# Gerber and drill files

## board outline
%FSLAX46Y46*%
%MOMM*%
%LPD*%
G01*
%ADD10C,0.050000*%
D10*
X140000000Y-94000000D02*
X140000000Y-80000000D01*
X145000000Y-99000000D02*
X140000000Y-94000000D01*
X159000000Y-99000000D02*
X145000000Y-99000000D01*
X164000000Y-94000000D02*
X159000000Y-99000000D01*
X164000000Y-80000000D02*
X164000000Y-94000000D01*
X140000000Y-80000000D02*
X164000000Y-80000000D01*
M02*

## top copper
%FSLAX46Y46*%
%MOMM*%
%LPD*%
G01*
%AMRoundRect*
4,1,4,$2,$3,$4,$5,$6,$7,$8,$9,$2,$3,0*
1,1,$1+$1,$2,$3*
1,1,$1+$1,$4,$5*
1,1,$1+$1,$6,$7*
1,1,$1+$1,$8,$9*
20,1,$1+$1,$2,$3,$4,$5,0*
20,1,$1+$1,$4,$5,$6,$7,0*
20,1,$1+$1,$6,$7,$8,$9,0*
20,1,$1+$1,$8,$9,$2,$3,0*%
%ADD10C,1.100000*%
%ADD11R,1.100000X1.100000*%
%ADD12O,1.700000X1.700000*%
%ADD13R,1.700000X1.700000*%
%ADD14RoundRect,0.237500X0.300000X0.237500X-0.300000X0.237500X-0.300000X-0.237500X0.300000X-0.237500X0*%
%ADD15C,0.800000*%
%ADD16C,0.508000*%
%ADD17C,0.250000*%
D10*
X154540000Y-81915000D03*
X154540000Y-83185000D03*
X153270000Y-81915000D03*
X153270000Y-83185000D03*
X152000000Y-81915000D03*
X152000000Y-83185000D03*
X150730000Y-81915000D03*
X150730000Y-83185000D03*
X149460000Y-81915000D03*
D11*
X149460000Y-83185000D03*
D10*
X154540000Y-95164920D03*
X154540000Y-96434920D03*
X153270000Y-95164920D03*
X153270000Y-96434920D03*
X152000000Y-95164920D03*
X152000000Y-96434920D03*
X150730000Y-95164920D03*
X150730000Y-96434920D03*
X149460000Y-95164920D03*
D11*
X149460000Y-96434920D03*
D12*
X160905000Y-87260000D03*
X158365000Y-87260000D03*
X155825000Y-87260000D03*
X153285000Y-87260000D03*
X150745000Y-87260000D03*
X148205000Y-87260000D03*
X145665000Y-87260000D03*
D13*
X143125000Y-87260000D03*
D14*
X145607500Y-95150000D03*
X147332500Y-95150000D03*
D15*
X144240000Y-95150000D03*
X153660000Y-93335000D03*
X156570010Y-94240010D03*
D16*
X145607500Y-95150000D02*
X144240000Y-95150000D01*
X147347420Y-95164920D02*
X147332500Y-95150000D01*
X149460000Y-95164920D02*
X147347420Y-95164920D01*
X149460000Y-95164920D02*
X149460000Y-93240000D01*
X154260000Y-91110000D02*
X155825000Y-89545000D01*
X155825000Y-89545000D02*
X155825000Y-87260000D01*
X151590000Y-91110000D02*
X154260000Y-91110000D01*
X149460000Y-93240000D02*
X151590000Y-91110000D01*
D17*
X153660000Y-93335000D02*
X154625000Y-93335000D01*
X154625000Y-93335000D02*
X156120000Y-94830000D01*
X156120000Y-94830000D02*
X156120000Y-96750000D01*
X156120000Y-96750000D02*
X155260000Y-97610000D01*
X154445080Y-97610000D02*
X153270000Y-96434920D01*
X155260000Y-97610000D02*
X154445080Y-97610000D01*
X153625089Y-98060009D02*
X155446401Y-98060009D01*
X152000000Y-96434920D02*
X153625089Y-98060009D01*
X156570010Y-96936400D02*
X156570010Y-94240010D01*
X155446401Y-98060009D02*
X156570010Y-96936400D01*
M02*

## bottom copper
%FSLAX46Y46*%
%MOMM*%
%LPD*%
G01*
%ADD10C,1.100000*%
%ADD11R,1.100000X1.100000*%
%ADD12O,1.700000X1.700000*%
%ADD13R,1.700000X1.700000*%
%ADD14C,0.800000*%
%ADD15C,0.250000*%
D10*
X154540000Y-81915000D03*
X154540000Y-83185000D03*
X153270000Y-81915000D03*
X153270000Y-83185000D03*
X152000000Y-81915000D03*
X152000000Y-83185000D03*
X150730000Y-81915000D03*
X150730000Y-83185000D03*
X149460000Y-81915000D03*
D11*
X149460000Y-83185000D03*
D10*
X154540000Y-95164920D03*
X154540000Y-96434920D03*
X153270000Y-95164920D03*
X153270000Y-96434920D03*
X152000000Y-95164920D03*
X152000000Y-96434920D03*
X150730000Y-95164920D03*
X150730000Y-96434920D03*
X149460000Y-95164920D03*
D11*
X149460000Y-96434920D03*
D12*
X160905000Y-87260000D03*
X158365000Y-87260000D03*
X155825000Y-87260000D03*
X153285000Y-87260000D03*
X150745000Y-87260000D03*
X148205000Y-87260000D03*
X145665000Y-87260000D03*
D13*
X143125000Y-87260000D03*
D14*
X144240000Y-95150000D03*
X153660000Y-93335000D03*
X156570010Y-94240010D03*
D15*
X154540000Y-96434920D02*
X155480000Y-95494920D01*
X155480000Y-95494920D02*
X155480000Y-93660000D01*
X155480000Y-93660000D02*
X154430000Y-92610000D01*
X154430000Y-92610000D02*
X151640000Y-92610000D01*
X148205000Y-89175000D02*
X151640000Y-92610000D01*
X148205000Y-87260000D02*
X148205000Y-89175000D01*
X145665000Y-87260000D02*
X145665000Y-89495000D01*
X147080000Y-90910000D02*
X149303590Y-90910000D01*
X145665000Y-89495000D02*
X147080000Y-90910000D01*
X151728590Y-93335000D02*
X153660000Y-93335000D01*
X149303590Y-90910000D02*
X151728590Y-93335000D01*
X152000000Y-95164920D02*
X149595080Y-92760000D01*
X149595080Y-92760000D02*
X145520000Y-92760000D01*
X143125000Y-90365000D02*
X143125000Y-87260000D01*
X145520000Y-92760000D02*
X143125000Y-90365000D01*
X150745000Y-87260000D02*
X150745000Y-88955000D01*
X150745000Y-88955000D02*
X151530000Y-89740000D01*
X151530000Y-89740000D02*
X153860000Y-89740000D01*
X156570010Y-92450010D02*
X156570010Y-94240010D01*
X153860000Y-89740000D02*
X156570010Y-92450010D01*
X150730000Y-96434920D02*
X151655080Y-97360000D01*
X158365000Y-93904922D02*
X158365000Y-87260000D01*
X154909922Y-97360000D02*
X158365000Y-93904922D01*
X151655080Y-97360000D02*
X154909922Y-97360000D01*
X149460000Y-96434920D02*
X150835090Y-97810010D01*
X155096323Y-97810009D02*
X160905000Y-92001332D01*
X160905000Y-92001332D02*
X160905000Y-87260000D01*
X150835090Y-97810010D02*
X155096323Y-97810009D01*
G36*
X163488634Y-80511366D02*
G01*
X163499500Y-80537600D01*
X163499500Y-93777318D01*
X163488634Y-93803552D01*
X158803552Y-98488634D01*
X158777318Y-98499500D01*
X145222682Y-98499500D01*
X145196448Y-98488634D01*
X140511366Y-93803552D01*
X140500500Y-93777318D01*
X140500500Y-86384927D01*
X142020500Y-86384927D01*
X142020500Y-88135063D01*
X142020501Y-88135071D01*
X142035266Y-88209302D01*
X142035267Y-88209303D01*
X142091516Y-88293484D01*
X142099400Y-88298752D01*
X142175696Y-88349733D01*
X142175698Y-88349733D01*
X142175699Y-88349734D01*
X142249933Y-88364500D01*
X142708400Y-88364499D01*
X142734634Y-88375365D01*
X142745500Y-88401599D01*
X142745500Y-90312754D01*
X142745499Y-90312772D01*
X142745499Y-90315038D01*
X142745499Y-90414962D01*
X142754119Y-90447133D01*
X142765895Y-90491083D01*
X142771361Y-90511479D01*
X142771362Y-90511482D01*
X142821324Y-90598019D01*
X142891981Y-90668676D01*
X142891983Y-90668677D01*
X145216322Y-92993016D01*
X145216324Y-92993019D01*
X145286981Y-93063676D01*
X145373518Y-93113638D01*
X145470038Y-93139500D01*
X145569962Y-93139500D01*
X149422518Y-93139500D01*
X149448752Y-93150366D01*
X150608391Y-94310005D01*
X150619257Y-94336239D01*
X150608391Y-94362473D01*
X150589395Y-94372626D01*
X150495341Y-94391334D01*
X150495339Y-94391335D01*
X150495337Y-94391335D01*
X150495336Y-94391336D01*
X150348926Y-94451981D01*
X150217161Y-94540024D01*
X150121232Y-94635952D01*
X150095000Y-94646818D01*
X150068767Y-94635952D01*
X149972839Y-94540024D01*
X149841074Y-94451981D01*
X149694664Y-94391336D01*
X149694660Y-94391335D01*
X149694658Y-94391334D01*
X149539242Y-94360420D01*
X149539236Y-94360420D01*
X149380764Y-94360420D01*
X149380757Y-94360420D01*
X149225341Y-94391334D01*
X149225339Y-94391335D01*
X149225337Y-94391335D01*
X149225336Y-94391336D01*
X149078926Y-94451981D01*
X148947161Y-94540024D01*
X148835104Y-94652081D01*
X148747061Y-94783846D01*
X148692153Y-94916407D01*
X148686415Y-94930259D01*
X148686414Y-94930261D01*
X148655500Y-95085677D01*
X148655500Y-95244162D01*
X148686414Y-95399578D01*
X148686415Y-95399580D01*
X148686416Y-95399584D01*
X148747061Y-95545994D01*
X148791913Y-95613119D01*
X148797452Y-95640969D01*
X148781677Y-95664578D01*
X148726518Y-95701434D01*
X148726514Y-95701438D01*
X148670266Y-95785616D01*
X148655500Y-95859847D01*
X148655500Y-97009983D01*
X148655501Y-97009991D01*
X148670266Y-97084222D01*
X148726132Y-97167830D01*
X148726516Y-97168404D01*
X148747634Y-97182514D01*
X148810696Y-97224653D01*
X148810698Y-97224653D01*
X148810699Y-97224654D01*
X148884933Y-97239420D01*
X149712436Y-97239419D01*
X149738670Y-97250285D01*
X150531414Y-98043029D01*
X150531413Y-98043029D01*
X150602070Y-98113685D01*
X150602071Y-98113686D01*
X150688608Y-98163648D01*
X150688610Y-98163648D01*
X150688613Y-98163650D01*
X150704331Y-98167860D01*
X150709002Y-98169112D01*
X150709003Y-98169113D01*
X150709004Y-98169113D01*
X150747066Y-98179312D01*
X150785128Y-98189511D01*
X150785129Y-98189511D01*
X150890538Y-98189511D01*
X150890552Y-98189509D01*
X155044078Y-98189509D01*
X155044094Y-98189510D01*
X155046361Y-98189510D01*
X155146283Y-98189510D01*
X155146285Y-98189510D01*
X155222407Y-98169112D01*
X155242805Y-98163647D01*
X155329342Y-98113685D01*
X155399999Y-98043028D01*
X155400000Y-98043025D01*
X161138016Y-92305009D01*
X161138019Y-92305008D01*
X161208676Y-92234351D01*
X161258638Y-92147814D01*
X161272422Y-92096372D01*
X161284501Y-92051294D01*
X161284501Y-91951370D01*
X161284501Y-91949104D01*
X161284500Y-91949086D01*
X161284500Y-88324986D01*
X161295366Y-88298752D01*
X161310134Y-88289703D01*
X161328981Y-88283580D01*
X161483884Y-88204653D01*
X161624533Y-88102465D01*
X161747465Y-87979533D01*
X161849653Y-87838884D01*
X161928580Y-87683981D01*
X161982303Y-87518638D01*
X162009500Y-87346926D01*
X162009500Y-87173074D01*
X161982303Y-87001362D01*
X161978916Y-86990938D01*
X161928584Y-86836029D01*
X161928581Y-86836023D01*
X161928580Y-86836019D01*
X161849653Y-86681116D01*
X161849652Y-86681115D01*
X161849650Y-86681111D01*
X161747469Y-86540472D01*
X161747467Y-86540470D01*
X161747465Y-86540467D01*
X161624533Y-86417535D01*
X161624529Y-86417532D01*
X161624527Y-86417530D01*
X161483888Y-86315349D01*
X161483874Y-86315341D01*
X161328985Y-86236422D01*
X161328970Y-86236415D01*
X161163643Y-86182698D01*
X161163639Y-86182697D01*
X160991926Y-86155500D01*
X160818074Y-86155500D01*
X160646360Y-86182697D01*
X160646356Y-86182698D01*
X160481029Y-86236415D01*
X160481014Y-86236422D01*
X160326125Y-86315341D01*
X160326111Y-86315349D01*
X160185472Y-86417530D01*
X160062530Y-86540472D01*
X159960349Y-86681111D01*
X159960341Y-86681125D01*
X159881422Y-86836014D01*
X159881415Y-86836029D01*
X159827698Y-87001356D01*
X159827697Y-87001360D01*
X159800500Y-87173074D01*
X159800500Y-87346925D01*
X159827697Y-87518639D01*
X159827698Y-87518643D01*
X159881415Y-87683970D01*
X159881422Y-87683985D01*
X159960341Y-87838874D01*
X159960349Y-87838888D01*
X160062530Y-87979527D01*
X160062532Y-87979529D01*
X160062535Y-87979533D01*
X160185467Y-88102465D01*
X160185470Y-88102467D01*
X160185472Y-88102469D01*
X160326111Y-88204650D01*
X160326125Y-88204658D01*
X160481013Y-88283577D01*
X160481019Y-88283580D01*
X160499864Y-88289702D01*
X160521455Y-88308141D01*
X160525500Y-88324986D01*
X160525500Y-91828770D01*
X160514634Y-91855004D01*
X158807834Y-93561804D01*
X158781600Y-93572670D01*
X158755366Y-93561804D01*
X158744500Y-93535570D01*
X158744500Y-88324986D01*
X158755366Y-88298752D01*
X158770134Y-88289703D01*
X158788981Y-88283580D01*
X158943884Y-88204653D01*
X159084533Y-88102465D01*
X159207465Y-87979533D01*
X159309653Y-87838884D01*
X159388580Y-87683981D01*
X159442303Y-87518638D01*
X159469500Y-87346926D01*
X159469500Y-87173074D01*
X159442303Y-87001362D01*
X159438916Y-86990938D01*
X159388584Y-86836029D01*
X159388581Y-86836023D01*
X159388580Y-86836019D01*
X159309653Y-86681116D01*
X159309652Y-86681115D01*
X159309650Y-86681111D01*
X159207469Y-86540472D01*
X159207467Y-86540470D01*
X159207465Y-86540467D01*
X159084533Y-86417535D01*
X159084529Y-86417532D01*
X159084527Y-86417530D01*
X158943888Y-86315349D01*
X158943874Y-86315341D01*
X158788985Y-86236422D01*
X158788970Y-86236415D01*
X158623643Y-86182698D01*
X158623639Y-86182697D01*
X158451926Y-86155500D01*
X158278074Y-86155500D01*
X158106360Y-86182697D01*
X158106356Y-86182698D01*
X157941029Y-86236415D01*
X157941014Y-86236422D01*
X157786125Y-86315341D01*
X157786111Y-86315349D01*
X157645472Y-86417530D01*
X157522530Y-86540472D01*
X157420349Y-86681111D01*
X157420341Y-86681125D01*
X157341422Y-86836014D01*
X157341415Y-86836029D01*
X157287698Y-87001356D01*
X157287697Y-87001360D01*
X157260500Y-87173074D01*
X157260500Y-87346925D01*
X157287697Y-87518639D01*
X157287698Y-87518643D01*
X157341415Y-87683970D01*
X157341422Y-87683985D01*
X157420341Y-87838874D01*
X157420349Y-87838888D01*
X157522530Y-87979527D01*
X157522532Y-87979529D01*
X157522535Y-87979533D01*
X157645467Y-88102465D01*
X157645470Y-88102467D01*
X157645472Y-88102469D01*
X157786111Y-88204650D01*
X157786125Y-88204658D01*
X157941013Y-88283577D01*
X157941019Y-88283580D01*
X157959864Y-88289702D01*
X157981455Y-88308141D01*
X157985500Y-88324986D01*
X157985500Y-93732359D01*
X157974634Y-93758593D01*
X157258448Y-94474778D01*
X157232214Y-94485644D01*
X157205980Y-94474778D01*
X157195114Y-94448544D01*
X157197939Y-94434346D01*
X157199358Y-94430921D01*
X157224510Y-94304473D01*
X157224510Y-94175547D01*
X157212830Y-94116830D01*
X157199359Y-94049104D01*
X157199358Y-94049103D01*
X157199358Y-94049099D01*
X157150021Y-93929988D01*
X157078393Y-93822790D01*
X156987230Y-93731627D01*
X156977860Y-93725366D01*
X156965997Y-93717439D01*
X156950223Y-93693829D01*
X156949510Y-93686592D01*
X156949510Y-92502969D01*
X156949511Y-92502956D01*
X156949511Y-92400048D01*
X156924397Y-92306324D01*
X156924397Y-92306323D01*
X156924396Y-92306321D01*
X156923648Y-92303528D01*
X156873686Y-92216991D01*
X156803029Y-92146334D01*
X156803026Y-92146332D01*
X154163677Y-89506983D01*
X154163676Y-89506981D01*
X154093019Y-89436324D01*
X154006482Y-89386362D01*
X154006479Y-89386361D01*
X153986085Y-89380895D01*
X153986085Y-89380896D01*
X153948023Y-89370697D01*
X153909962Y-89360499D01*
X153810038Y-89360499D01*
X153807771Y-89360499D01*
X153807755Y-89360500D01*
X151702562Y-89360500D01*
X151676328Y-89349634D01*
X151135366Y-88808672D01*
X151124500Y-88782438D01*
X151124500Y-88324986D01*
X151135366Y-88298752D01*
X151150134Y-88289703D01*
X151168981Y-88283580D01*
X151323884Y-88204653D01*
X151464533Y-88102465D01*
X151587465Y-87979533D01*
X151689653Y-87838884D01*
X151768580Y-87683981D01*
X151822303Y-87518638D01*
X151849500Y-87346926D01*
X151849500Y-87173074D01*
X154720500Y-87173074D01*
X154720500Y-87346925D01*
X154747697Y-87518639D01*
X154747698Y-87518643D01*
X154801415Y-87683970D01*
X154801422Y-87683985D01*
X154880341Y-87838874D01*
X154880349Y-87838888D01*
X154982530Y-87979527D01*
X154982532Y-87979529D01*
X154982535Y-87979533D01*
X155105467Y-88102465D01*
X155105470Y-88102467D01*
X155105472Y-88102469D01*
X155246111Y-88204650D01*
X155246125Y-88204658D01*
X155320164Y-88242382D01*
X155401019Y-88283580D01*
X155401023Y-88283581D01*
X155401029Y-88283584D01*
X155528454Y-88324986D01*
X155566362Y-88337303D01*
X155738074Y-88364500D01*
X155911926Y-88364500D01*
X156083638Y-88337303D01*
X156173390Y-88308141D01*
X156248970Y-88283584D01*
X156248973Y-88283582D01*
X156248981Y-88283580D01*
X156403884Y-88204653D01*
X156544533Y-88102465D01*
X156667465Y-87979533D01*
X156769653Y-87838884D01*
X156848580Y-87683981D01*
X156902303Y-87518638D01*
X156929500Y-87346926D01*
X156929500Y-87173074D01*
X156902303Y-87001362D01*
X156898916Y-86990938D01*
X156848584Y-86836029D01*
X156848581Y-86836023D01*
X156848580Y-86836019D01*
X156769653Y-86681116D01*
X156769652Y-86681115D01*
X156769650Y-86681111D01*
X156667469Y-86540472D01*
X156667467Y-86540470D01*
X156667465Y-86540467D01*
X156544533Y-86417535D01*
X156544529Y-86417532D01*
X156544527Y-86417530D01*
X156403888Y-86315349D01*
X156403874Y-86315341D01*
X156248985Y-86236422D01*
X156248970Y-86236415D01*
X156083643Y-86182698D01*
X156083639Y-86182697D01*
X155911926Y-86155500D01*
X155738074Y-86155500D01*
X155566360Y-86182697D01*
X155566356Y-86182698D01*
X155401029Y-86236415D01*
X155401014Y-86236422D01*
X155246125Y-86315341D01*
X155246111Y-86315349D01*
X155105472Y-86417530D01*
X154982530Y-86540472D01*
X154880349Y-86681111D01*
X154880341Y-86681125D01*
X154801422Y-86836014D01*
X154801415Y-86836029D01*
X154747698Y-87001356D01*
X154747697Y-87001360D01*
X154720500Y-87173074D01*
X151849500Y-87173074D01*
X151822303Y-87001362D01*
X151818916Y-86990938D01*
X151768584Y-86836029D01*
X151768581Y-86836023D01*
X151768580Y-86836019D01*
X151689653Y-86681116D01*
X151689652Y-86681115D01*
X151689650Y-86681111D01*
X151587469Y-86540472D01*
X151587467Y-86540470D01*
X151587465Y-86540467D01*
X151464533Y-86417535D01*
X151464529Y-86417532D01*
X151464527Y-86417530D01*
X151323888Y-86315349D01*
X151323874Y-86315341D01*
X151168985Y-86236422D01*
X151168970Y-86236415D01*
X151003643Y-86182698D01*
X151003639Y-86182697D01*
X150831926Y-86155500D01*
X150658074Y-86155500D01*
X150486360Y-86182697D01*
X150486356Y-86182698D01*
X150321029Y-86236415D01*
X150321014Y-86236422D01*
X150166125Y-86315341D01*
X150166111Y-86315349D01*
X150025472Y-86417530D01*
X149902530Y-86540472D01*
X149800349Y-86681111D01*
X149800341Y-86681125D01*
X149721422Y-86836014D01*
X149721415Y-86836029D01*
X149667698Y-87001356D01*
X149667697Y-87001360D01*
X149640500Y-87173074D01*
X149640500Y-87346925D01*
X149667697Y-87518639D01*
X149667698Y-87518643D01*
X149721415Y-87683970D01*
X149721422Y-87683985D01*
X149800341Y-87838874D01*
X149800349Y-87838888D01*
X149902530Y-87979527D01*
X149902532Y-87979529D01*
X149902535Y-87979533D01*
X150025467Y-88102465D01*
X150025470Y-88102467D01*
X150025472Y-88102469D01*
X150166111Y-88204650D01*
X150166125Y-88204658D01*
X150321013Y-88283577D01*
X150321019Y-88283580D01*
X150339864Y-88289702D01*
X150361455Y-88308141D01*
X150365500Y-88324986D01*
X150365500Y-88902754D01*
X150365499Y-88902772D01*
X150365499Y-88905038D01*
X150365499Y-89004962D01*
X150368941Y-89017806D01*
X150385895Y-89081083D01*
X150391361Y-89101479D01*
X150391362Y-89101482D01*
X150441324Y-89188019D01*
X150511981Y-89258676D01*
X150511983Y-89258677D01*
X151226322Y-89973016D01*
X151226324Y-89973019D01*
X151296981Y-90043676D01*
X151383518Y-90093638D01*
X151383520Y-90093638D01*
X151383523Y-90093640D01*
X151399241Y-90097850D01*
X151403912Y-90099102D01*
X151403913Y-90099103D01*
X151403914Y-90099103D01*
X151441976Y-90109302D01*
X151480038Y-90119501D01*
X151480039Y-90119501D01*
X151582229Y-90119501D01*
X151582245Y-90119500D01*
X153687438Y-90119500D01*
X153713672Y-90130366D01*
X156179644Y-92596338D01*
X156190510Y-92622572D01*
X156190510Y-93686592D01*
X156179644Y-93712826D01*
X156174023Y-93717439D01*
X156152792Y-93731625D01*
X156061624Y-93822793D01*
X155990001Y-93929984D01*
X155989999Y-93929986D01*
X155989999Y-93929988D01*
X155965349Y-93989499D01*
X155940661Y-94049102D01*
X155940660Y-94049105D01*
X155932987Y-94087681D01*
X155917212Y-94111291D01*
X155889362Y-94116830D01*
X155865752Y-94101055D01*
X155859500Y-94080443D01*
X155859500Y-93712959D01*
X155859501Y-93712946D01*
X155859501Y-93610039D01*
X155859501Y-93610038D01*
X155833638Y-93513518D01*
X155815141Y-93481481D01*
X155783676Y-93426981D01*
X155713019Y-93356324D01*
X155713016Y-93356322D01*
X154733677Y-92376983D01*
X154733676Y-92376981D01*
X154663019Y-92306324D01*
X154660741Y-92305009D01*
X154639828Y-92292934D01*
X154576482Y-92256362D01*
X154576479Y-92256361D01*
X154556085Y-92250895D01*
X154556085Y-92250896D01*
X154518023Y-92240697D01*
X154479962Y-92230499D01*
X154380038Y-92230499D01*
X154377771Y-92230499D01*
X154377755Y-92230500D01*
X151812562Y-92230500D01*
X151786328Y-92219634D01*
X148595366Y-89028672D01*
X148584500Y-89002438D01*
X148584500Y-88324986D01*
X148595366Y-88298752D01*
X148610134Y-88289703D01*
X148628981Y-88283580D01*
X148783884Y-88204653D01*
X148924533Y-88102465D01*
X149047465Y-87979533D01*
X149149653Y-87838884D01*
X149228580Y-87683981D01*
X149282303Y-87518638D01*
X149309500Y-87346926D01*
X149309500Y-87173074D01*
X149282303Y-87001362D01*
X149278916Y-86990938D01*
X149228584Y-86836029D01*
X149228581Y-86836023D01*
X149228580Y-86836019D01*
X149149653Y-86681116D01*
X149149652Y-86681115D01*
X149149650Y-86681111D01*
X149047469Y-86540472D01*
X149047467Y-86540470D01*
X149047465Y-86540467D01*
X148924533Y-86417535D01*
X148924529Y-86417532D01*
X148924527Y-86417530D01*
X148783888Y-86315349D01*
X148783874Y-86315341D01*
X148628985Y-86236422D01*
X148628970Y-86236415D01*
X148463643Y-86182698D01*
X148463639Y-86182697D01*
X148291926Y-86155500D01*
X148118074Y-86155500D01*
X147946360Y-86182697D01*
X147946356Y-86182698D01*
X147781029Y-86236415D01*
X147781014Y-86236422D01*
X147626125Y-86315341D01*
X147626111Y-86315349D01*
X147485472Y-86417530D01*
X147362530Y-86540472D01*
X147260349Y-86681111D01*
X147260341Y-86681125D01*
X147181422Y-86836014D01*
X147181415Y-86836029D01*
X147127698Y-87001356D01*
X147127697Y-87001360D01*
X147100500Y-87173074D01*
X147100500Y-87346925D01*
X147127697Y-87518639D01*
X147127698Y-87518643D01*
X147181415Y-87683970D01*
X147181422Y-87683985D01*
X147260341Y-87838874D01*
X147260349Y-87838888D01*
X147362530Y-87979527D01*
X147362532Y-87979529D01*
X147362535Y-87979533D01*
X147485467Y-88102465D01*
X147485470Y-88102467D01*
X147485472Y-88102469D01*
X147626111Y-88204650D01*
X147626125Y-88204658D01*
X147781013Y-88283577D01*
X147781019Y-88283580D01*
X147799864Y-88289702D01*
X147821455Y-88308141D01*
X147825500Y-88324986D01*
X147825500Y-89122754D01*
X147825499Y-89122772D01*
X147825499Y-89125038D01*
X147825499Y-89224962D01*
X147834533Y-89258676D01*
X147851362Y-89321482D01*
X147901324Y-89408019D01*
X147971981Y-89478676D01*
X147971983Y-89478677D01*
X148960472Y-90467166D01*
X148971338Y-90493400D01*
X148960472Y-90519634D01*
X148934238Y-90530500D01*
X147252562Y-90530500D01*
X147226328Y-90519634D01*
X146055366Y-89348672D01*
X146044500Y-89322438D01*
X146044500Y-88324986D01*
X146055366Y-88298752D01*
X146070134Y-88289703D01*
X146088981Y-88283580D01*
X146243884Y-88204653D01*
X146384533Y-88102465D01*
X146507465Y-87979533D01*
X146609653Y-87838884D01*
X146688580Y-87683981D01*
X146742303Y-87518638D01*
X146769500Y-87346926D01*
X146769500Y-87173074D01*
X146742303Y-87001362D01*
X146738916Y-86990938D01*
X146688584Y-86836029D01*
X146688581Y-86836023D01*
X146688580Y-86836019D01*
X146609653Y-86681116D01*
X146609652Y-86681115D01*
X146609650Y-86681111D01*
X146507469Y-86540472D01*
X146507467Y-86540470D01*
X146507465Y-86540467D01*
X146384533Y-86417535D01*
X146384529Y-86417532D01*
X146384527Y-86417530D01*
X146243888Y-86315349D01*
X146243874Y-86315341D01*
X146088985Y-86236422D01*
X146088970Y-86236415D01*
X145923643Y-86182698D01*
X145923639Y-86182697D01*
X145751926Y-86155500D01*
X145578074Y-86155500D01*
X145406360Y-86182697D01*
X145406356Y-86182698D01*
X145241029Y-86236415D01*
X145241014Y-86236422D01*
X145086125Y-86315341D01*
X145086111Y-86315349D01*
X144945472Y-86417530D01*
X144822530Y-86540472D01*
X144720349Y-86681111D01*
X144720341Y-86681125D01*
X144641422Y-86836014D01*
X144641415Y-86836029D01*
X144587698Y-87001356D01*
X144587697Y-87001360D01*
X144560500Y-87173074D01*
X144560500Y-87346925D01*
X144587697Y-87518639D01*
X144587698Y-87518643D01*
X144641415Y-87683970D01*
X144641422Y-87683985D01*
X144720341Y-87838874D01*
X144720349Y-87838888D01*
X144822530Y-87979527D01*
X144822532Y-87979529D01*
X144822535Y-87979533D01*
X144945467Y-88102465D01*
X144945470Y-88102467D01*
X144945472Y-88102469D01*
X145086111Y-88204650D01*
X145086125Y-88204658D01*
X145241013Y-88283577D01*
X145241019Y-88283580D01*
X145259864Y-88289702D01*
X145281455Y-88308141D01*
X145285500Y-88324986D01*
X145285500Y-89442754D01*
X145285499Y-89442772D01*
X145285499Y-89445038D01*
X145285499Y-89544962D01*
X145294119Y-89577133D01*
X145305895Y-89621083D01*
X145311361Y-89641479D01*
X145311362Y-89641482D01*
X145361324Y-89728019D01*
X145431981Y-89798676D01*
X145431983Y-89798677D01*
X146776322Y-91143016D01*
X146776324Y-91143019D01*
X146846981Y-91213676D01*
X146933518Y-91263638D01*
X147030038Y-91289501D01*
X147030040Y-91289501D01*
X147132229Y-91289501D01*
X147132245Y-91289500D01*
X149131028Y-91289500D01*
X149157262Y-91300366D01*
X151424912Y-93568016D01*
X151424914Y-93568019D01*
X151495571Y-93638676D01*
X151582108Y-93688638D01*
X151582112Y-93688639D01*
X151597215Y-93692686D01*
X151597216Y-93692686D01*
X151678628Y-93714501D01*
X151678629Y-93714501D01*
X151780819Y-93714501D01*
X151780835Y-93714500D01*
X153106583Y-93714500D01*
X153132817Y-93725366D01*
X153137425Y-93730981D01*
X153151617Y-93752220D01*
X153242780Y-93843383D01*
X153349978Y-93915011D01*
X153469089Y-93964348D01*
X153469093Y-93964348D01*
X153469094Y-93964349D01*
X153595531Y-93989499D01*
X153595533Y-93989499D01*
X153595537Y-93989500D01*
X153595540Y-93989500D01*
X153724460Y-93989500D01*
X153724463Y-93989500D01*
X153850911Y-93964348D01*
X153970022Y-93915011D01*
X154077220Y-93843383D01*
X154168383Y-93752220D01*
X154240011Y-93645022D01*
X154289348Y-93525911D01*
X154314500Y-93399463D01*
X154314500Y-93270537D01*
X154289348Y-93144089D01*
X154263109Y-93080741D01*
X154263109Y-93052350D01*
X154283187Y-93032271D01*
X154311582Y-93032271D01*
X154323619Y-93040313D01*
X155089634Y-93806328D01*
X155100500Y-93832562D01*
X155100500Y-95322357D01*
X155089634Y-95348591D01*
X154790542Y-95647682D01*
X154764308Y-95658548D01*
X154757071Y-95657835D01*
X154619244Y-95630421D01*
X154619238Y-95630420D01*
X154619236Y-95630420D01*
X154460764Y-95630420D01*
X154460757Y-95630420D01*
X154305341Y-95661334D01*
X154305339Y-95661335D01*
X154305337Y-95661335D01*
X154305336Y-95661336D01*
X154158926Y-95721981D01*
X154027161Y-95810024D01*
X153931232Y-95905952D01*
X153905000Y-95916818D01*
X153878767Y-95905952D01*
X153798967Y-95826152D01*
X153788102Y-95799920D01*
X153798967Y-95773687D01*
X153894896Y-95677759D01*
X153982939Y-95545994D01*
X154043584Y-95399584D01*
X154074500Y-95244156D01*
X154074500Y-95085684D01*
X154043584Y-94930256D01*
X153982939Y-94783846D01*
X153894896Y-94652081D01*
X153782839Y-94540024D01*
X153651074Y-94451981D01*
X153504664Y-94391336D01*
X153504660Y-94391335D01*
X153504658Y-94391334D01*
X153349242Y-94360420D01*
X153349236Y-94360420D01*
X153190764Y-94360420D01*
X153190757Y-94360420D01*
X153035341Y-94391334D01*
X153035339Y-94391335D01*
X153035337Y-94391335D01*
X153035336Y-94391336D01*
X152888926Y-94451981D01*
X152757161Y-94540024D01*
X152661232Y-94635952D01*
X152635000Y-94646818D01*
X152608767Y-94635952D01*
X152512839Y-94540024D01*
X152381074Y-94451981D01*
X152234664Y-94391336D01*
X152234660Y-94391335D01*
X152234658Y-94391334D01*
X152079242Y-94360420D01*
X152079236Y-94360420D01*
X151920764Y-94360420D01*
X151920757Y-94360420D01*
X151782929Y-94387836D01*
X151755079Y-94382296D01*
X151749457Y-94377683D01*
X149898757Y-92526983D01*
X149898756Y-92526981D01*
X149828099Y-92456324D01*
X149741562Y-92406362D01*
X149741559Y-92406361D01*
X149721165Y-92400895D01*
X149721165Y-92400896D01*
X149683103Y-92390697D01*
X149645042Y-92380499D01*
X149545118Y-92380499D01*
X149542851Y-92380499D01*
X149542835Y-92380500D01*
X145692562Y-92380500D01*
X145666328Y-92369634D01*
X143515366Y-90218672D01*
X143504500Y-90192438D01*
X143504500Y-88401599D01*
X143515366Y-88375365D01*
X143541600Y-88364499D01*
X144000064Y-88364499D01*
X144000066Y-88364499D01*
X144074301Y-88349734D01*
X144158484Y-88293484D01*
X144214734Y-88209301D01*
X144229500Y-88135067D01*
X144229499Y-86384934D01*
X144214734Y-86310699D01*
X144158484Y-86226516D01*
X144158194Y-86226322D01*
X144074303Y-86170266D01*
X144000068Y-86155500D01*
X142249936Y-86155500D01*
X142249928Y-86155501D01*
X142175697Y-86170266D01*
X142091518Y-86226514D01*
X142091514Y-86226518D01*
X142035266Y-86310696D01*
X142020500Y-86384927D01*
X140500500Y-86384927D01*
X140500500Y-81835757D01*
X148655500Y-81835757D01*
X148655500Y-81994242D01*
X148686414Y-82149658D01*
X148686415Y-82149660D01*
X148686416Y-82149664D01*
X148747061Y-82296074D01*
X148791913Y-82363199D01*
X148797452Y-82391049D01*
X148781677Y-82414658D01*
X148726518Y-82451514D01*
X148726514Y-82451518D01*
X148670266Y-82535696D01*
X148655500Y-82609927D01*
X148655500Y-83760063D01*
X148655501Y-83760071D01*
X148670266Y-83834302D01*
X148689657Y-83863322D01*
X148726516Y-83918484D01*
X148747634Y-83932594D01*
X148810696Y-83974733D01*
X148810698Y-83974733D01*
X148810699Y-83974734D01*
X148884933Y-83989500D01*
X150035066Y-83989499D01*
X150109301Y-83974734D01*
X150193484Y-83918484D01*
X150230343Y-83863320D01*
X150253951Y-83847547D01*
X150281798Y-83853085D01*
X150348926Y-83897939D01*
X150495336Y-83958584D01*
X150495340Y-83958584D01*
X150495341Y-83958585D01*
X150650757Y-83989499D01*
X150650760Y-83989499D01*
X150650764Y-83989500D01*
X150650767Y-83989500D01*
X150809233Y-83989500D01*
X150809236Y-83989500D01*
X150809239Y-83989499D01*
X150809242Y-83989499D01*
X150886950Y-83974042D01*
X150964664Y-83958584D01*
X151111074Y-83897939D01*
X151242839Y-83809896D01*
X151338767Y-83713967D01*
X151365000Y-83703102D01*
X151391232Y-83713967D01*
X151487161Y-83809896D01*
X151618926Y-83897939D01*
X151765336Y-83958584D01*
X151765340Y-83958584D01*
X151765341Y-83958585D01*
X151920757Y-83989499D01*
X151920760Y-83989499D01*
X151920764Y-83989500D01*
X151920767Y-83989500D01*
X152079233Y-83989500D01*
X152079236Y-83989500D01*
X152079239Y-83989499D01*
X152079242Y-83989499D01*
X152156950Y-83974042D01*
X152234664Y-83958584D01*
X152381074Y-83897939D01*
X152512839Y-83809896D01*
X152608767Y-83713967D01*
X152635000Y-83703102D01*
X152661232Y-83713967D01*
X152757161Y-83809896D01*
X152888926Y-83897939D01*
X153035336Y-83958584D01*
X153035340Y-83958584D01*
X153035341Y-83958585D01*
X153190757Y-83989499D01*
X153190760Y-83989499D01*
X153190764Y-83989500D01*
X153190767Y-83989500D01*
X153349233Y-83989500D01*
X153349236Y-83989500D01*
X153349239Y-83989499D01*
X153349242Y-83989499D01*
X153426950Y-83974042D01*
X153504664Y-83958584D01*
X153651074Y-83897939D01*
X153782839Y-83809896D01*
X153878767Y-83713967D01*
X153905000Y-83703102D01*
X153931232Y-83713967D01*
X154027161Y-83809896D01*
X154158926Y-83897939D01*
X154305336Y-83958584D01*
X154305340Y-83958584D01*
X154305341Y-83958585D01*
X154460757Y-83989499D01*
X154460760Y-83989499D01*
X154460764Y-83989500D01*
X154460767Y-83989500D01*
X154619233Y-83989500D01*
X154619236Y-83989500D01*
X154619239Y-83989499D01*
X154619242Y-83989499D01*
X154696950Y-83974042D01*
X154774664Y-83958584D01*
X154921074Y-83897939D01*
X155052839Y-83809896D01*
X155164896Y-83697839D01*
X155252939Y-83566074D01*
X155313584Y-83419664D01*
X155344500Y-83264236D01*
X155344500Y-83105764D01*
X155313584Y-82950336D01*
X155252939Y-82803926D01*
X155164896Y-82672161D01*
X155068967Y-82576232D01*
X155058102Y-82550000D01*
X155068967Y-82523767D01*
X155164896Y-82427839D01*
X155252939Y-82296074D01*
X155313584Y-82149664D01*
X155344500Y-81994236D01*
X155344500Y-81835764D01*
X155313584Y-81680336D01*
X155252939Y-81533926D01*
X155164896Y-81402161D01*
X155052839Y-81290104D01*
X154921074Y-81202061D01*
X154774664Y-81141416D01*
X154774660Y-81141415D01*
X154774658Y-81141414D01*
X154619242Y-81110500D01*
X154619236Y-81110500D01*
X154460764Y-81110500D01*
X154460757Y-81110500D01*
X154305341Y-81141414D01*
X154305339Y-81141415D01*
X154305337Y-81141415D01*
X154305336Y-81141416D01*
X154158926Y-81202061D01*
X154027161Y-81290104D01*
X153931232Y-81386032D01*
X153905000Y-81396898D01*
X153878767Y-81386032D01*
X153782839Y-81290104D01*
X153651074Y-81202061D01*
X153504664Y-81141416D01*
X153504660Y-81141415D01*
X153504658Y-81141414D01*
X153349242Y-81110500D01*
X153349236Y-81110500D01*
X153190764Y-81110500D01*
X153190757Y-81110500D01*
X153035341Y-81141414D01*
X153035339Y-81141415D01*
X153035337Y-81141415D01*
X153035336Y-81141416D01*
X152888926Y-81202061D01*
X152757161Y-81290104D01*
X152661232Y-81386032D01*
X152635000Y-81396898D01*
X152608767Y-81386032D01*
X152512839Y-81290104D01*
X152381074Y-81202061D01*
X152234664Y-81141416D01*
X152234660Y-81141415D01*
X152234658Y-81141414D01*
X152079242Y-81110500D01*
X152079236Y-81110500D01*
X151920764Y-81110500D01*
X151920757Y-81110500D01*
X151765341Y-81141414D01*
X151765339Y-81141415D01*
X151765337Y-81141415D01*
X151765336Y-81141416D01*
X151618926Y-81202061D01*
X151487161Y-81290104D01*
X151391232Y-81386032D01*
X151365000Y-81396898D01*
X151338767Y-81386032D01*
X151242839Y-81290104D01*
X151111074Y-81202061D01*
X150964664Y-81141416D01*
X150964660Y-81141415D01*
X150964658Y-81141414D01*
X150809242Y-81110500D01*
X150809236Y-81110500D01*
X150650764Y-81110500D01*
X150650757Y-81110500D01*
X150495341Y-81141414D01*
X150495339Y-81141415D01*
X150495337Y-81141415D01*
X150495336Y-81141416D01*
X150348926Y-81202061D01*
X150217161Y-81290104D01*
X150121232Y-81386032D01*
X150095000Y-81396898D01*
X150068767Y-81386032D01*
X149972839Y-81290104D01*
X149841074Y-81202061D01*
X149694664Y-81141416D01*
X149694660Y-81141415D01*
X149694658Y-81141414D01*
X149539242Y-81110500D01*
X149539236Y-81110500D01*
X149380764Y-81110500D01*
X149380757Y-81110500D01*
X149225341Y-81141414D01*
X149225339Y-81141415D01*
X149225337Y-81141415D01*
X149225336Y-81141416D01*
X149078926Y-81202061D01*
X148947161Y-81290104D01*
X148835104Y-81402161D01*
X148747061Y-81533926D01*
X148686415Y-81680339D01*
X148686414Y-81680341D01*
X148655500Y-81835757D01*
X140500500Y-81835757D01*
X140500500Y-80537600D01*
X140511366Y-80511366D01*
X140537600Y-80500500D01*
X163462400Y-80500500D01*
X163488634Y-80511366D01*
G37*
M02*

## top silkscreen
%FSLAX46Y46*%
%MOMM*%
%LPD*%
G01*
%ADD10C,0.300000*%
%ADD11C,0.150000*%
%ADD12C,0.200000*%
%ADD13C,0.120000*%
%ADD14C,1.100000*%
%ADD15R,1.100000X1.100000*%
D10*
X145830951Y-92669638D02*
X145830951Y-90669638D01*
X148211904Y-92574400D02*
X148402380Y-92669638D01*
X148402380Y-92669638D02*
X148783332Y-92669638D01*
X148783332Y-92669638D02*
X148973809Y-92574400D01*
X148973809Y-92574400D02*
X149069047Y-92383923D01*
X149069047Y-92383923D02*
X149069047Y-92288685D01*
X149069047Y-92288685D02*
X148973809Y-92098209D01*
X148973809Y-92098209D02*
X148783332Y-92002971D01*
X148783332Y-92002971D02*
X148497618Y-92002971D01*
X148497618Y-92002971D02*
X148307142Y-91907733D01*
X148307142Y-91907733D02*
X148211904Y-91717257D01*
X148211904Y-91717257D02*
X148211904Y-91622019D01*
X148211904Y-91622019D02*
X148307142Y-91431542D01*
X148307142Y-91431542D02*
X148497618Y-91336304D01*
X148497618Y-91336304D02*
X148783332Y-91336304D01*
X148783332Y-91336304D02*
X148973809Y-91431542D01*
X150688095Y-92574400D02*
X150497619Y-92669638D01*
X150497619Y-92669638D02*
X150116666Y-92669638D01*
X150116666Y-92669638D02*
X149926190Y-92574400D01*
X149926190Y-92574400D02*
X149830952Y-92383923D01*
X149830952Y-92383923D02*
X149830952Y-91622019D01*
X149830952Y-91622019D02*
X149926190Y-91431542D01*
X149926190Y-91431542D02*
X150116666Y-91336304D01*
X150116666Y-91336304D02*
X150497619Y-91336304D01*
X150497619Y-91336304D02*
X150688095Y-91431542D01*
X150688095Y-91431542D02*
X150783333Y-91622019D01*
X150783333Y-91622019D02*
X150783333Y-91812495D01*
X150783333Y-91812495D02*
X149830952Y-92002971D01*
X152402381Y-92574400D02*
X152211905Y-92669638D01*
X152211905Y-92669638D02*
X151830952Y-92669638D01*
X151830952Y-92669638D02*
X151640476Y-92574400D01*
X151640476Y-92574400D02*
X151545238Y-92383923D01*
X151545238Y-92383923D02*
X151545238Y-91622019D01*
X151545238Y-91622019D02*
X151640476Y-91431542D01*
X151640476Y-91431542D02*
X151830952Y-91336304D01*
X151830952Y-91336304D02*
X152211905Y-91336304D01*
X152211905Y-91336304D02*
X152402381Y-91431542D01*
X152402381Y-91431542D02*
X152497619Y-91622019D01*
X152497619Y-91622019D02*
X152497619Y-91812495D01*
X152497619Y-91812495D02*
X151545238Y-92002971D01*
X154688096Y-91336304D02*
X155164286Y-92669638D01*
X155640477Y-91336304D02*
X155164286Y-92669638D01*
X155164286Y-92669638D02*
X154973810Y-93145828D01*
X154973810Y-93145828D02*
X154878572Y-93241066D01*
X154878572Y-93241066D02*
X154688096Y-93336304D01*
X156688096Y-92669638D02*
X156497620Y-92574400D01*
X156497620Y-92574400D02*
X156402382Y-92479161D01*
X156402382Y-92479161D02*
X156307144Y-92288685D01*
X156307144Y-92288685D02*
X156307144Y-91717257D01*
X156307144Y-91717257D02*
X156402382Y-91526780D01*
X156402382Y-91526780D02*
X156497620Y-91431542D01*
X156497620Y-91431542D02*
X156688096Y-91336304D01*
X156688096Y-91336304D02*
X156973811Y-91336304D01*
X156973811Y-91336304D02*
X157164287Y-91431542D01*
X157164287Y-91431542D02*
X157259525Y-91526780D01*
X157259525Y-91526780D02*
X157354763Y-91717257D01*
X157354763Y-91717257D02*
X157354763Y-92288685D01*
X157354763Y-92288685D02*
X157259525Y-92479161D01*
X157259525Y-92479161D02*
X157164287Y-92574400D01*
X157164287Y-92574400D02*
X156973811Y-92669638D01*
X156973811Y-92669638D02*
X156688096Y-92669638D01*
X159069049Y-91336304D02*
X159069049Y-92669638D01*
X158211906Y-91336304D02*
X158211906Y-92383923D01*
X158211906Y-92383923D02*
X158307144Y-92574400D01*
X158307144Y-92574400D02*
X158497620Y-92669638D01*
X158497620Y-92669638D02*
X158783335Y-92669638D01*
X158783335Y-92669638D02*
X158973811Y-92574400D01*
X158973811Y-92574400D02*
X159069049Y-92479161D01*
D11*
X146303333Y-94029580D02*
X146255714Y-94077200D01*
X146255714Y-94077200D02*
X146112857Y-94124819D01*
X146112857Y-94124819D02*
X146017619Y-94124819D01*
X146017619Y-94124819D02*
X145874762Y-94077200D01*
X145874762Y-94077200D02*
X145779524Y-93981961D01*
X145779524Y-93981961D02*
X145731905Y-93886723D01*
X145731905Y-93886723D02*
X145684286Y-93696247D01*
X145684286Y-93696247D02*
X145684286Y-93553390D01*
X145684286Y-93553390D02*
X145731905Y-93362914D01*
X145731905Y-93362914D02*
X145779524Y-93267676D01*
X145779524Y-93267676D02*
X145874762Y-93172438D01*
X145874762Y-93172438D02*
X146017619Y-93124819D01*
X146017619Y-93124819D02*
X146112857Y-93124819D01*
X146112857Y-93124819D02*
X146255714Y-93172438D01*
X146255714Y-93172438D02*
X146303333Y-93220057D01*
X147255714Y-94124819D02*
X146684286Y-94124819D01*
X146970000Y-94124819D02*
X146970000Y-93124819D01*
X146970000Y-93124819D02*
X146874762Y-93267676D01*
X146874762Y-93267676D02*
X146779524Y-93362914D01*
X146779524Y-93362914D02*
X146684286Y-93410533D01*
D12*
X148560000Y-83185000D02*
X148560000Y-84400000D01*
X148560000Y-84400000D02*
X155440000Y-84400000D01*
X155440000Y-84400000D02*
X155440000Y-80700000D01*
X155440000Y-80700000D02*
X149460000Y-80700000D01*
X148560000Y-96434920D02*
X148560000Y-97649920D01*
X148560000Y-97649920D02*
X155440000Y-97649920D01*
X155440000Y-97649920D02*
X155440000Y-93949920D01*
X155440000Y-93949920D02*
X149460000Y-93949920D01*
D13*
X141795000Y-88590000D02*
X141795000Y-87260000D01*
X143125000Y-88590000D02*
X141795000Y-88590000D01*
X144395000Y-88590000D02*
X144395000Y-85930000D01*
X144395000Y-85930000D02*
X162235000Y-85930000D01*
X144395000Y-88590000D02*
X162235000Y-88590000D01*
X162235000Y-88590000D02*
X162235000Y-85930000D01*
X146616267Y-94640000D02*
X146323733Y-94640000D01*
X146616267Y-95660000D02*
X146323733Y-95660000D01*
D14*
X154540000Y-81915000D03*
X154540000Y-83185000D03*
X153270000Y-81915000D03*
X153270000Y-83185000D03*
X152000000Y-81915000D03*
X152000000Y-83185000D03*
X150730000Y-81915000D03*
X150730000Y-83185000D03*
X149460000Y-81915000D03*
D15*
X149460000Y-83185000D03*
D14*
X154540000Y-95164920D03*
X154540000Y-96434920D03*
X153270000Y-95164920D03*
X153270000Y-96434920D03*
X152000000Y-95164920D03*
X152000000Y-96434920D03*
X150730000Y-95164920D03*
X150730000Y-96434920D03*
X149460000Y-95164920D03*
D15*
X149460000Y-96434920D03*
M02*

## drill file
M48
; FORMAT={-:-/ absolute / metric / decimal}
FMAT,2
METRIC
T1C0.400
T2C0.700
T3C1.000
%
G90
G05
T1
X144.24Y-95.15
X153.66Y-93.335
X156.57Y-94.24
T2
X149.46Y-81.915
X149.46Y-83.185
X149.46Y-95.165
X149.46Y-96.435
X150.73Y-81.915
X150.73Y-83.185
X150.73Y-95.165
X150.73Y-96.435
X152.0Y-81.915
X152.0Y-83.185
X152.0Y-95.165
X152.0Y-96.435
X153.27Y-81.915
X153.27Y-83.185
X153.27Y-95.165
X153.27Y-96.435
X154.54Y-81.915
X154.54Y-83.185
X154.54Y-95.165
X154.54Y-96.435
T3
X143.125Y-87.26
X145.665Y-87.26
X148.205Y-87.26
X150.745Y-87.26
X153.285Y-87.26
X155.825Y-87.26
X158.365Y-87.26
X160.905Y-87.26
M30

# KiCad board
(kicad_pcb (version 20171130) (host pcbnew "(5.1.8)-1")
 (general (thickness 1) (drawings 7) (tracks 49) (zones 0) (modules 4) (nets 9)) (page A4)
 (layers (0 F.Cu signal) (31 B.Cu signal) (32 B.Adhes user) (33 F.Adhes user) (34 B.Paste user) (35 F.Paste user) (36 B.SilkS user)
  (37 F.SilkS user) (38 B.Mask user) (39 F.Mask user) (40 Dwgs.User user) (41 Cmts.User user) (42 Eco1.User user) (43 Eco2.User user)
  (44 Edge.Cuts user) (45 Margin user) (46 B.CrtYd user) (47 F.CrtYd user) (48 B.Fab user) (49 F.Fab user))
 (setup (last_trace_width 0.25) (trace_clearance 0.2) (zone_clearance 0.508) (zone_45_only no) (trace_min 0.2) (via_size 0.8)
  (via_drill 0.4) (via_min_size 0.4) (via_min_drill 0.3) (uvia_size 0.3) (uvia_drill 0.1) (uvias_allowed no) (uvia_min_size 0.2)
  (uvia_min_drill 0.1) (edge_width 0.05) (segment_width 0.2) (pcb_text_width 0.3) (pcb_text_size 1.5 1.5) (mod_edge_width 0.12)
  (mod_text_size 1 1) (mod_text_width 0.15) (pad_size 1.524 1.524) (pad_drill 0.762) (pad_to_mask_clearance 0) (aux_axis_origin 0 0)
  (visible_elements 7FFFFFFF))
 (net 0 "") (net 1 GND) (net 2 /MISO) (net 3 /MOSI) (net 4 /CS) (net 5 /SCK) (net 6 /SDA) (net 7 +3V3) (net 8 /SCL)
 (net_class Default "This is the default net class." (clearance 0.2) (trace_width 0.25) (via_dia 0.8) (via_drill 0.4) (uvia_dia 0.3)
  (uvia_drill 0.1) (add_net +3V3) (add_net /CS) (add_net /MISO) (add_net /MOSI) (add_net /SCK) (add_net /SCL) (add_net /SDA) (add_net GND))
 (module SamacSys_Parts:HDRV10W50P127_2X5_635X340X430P (layer F.Cu) (at 152 82.55)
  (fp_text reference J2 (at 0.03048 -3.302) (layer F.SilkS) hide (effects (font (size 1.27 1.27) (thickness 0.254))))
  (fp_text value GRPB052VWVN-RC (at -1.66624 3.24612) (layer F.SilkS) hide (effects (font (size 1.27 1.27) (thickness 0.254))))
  (fp_line (start -3.44 0.635) (end -3.44 1.85) (layer F.SilkS) (width 0.2))
  (fp_line (start -3.44 1.85) (end 3.44 1.85) (layer F.SilkS) (width 0.2))
  (fp_line (start 3.44 1.85) (end 3.44 -1.85) (layer F.SilkS) (width 0.2))
  (fp_line (start 3.44 -1.85) (end -2.54 -1.85) (layer F.SilkS) (width 0.2))
  (pad 10 thru_hole circle (at 2.54 -0.635 90) (size 1.1 1.1) (drill 0.7) (layers *.Cu *.Mask F.SilkS))
  (pad 9 thru_hole circle (at 2.54 0.635 90) (size 1.1 1.1) (drill 0.7) (layers *.Cu *.Mask F.SilkS))
  (pad 8 thru_hole circle (at 1.27 -0.635 90) (size 1.1 1.1) (drill 0.7) (layers *.Cu *.Mask F.SilkS))
  (pad 7 thru_hole circle (at 1.27 0.635 90) (size 1.1 1.1) (drill 0.7) (layers *.Cu *.Mask F.SilkS))
  (pad 6 thru_hole circle (at 0 -0.635 90) (size 1.1 1.1) (drill 0.7) (layers *.Cu *.Mask F.SilkS))
  (pad 5 thru_hole circle (at 0 0.635 90) (size 1.1 1.1) (drill 0.7) (layers *.Cu *.Mask F.SilkS))
  (pad 4 thru_hole circle (at -1.27 -0.635 90) (size 1.1 1.1) (drill 0.7) (layers *.Cu *.Mask F.SilkS))
  (pad 3 thru_hole circle (at -1.27 0.635 90) (size 1.1 1.1) (drill 0.7) (layers *.Cu *.Mask F.SilkS))
  (pad 2 thru_hole circle (at -2.54 -0.635 90) (size 1.1 1.1) (drill 0.7) (layers *.Cu *.Mask F.SilkS))
  (pad 1 thru_hole rect (at -2.54 0.635 90) (size 1.1 1.1) (drill 0.7) (layers *.Cu *.Mask F.SilkS)))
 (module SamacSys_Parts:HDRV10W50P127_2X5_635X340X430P (layer F.Cu) (at 152 95.8)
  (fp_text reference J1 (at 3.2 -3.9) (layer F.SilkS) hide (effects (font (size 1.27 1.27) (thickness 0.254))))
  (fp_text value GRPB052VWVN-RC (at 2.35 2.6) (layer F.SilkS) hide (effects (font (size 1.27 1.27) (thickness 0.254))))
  (fp_line (start -3.44 0.63492) (end -3.44 1.84992) (layer F.SilkS) (width 0.2))
  (fp_line (start -3.44 1.84992) (end 3.44 1.84992) (layer F.SilkS) (width 0.2))
  (fp_line (start 3.44 1.84992) (end 3.44 -1.85008) (layer F.SilkS) (width 0.2))
  (fp_line (start 3.44 -1.85008) (end -2.54 -1.85008) (layer F.SilkS) (width 0.2))
  (pad 10 thru_hole circle (at 2.54 -0.63508 90) (size 1.1 1.1) (drill 0.7) (layers *.Cu *.Mask F.SilkS) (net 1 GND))
  (pad 9 thru_hole circle (at 2.54 0.63492 90) (size 1.1 1.1) (drill 0.7) (layers *.Cu *.Mask F.SilkS) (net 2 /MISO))
  (pad 8 thru_hole circle (at 1.27 -0.63508 90) (size 1.1 1.1) (drill 0.7) (layers *.Cu *.Mask F.SilkS))
  (pad 7 thru_hole circle (at 1.27 0.63492 90) (size 1.1 1.1) (drill 0.7) (layers *.Cu *.Mask F.SilkS) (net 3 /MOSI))
  (pad 6 thru_hole circle (at 0 -0.63508 90) (size 1.1 1.1) (drill 0.7) (layers *.Cu *.Mask F.SilkS) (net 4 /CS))
  (pad 5 thru_hole circle (at 0 0.63492 90) (size 1.1 1.1) (drill 0.7) (layers *.Cu *.Mask F.SilkS) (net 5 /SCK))
  (pad 4 thru_hole circle (at -1.27 -0.63508 90) (size 1.1 1.1) (drill 0.7) (layers *.Cu *.Mask F.SilkS))
  (pad 3 thru_hole circle (at -1.27 0.63492 90) (size 1.1 1.1) (drill 0.7) (layers *.Cu *.Mask F.SilkS) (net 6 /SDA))
  (pad 2 thru_hole circle (at -2.54 -0.63508 90) (size 1.1 1.1) (drill 0.7) (layers *.Cu *.Mask F.SilkS) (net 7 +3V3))
  (pad 1 thru_hole rect (at -2.54 0.63492 90) (size 1.1 1.1) (drill 0.7) (layers *.Cu *.Mask F.SilkS) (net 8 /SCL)))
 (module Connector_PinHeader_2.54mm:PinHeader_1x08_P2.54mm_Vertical (layer F.Cu) (at 143.125 87.26 90)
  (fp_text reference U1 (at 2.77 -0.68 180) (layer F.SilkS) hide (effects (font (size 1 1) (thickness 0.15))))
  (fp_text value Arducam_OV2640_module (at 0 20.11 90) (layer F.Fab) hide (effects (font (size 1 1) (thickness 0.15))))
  (fp_line (start -1.33 -1.33) (end 0 -1.33) (layer F.SilkS) (width 0.12))
  (fp_line (start -1.33 0) (end -1.33 -1.33) (layer F.SilkS) (width 0.12))
  (fp_line (start -1.33 1.27) (end 1.33 1.27) (layer F.SilkS) (width 0.12))
  (fp_line (start 1.33 1.27) (end 1.33 19.11) (layer F.SilkS) (width 0.12))
  (fp_line (start -1.33 1.27) (end -1.33 19.11) (layer F.SilkS) (width 0.12))
  (fp_line (start -1.33 19.11) (end 1.33 19.11) (layer F.SilkS) (width 0.12))
  (pad 8 thru_hole oval (at 0 17.78 90) (size 1.7 1.7) (drill 1) (layers *.Cu *.Mask) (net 8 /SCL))
  (pad 7 thru_hole oval (at 0 15.24 90) (size 1.7 1.7) (drill 1) (layers *.Cu *.Mask) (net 6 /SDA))
  (pad 6 thru_hole oval (at 0 12.7 90) (size 1.7 1.7) (drill 1) (layers *.Cu *.Mask) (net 7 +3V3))
  (pad 5 thru_hole oval (at 0 10.16 90) (size 1.7 1.7) (drill 1) (layers *.Cu *.Mask) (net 1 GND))
  (pad 4 thru_hole oval (at 0 7.62 90) (size 1.7 1.7) (drill 1) (layers *.Cu *.Mask) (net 5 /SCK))
  (pad 3 thru_hole oval (at 0 5.08 90) (size 1.7 1.7) (drill 1) (layers *.Cu *.Mask) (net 2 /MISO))
  (pad 2 thru_hole oval (at 0 2.54 90) (size 1.7 1.7) (drill 1) (layers *.Cu *.Mask) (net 3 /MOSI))
  (pad 1 thru_hole rect (at 0 0 90) (size 1.7 1.7) (drill 1) (layers *.Cu *.Mask) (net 4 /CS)))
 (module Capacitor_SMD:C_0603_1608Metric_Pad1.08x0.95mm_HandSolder (layer F.Cu) (at 146.47 95.15 180)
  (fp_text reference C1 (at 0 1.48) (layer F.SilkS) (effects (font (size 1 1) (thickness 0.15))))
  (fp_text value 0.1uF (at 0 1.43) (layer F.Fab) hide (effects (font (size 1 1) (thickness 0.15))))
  (fp_line (start -0.146267 0.51) (end 0.146267 0.51) (layer F.SilkS) (width 0.12))
  (fp_line (start -0.146267 -0.51) (end 0.146267 -0.51) (layer F.SilkS) (width 0.12))
  (pad 2 smd roundrect (at 0.8625 0 180) (size 1.075 0.95) (layers F.Cu F.Paste F.Mask) (roundrect_rratio 0.25) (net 1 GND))
  (pad 1 smd roundrect (at -0.8625 0 180) (size 1.075 0.95) (layers F.Cu F.Paste F.Mask) (roundrect_rratio 0.25) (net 7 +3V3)))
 (gr_line (start 140 94) (end 140 80) (layer Edge.Cuts) (width 0.05))
 (gr_line (start 145 99) (end 140 94) (layer Edge.Cuts) (width 0.05))
 (gr_line (start 159 99) (end 145 99) (layer Edge.Cuts) (width 0.05))
 (gr_line (start 164 94) (end 159 99) (layer Edge.Cuts) (width 0.05))
 (gr_line (start 164 80) (end 164 94) (layer Edge.Cuts) (width 0.05))
 (gr_line (start 140 80) (end 164 80) (layer Edge.Cuts) (width 0.05))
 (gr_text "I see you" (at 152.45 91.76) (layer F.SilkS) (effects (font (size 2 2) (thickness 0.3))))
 (via (at 144.24 95.15) (size 0.8) (drill 0.4) (layers F.Cu B.Cu) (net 1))
 (segment (start 145.6075 95.15) (end 144.24 95.15) (width 0.508) (layer F.Cu) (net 1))
 (segment (start 147.34742 95.16492) (end 147.3325 95.15) (width 0.508) (layer F.Cu) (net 7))
 (segment (start 149.46 95.16492) (end 147.34742 95.16492) (width 0.508) (layer F.Cu) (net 7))
 (segment (start 149.46 95.16492) (end 149.46 93.24) (width 0.508) (layer F.Cu) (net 7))
 (segment (start 154.26 91.11) (end 155.825 89.545) (width 0.508) (layer F.Cu) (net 7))
 (segment (start 155.825 89.545) (end 155.825 87.26) (width 0.508) (layer F.Cu) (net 7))
 (segment (start 151.59 91.11) (end 154.26 91.11) (width 0.508) (layer F.Cu) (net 7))
 (segment (start 149.46 93.24) (end 151.59 91.11) (width 0.508) (layer F.Cu) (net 7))
 (segment (start 154.54 96.43492) (end 155.48 95.49492) (width 0.25) (layer B.Cu) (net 2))
 (segment (start 155.48 95.49492) (end 155.48 93.66) (width 0.25) (layer B.Cu) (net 2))
 (segment (start 155.48 93.66) (end 154.43 92.61) (width 0.25) (layer B.Cu) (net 2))
 (segment (start 154.43 92.61) (end 151.64 92.61) (width 0.25) (layer B.Cu) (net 2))
 (segment (start 148.205 89.175) (end 151.64 92.61) (width 0.25) (layer B.Cu) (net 2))
 (segment (start 148.205 87.26) (end 148.205 89.175) (width 0.25) (layer B.Cu) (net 2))
 (segment (start 145.665 87.26) (end 145.665 89.495) (width 0.25) (layer B.Cu) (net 3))
 (segment (start 147.08 90.91) (end 149.30359 90.91) (width 0.25) (layer B.Cu) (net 3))
 (segment (start 145.665 89.495) (end 147.08 90.91) (width 0.25) (layer B.Cu) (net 3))
 (via (at 153.66 93.335) (size 0.8) (drill 0.4) (layers F.Cu B.Cu) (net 3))
 (segment (start 151.72859 93.335) (end 153.66 93.335) (width 0.25) (layer B.Cu) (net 3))
 (segment (start 149.30359 90.91) (end 151.72859 93.335) (width 0.25) (layer B.Cu) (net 3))
 (segment (start 153.66 93.335) (end 154.625 93.335) (width 0.25) (layer F.Cu) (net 3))
 (segment (start 154.625 93.335) (end 156.12 94.83) (width 0.25) (layer F.Cu) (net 3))
 (segment (start 156.12 94.83) (end 156.12 96.75) (width 0.25) (layer F.Cu) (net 3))
 (segment (start 156.12 96.75) (end 155.26 97.61) (width 0.25) (layer F.Cu) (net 3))
 (segment (start 154.44508 97.61) (end 153.27 96.43492) (width 0.25) (layer F.Cu) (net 3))
 (segment (start 155.26 97.61) (end 154.44508 97.61) (width 0.25) (layer F.Cu) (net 3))
 (segment (start 152 95.16492) (end 149.59508 92.76) (width 0.25) (layer B.Cu) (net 4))
 (segment (start 149.59508 92.76) (end 145.52 92.76) (width 0.25) (layer B.Cu) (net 4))
 (segment (start 143.125 90.365) (end 143.125 87.26) (width 0.25) (layer B.Cu) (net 4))
 (segment (start 145.52 92.76) (end 143.125 90.365) (width 0.25) (layer B.Cu) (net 4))
 (segment (start 153.625089 98.060009) (end 155.446401 98.060009) (width 0.25) (layer F.Cu) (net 5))
 (segment (start 152 96.43492) (end 153.625089 98.060009) (width 0.25) (layer F.Cu) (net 5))
 (segment (start 156.57001 96.9364) (end 156.57001 94.24001) (width 0.25) (layer F.Cu) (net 5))
 (segment (start 155.446401 98.060009) (end 156.57001 96.9364) (width 0.25) (layer F.Cu) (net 5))
 (segment (start 150.745 87.26) (end 150.745 88.955) (width 0.25) (layer B.Cu) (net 5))
 (segment (start 150.745 88.955) (end 151.53 89.74) (width 0.25) (layer B.Cu) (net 5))
 (segment (start 151.53 89.74) (end 153.86 89.74) (width 0.25) (layer B.Cu) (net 5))
 (via (at 156.57001 94.24001) (size 0.8) (drill 0.4) (layers F.Cu B.Cu) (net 5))
 (segment (start 156.57001 92.45001) (end 156.57001 94.24001) (width 0.25) (layer B.Cu) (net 5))
 (segment (start 153.86 89.74) (end 156.57001 92.45001) (width 0.25) (layer B.Cu) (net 5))
 (segment (start 150.73 96.43492) (end 151.65508 97.36) (width 0.25) (layer B.Cu) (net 6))
 (segment (start 158.365 93.904922) (end 158.365 87.26) (width 0.25) (layer B.Cu) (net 6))
 (segment (start 154.909922 97.36) (end 158.365 93.904922) (width 0.25) (layer B.Cu) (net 6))
 (segment (start 151.65508 97.36) (end 154.909922 97.36) (width 0.25) (layer B.Cu) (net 6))
 (segment (start 149.46 96.43492) (end 150.83509 97.81001) (width 0.25) (layer B.Cu) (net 8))
 (segment (start 155.096323 97.810009) (end 160.905 92.001332) (width 0.25) (layer B.Cu) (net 8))
 (segment (start 160.905 92.001332) (end 160.905 87.26) (width 0.25) (layer B.Cu) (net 8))
 (segment (start 150.83509 97.81001) (end 155.096323 97.810009) (width 0.25) (layer B.Cu) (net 8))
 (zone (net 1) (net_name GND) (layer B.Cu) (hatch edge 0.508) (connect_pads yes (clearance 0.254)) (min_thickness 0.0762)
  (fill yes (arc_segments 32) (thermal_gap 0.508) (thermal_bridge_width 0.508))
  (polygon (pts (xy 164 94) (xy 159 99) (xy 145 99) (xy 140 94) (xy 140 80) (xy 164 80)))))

